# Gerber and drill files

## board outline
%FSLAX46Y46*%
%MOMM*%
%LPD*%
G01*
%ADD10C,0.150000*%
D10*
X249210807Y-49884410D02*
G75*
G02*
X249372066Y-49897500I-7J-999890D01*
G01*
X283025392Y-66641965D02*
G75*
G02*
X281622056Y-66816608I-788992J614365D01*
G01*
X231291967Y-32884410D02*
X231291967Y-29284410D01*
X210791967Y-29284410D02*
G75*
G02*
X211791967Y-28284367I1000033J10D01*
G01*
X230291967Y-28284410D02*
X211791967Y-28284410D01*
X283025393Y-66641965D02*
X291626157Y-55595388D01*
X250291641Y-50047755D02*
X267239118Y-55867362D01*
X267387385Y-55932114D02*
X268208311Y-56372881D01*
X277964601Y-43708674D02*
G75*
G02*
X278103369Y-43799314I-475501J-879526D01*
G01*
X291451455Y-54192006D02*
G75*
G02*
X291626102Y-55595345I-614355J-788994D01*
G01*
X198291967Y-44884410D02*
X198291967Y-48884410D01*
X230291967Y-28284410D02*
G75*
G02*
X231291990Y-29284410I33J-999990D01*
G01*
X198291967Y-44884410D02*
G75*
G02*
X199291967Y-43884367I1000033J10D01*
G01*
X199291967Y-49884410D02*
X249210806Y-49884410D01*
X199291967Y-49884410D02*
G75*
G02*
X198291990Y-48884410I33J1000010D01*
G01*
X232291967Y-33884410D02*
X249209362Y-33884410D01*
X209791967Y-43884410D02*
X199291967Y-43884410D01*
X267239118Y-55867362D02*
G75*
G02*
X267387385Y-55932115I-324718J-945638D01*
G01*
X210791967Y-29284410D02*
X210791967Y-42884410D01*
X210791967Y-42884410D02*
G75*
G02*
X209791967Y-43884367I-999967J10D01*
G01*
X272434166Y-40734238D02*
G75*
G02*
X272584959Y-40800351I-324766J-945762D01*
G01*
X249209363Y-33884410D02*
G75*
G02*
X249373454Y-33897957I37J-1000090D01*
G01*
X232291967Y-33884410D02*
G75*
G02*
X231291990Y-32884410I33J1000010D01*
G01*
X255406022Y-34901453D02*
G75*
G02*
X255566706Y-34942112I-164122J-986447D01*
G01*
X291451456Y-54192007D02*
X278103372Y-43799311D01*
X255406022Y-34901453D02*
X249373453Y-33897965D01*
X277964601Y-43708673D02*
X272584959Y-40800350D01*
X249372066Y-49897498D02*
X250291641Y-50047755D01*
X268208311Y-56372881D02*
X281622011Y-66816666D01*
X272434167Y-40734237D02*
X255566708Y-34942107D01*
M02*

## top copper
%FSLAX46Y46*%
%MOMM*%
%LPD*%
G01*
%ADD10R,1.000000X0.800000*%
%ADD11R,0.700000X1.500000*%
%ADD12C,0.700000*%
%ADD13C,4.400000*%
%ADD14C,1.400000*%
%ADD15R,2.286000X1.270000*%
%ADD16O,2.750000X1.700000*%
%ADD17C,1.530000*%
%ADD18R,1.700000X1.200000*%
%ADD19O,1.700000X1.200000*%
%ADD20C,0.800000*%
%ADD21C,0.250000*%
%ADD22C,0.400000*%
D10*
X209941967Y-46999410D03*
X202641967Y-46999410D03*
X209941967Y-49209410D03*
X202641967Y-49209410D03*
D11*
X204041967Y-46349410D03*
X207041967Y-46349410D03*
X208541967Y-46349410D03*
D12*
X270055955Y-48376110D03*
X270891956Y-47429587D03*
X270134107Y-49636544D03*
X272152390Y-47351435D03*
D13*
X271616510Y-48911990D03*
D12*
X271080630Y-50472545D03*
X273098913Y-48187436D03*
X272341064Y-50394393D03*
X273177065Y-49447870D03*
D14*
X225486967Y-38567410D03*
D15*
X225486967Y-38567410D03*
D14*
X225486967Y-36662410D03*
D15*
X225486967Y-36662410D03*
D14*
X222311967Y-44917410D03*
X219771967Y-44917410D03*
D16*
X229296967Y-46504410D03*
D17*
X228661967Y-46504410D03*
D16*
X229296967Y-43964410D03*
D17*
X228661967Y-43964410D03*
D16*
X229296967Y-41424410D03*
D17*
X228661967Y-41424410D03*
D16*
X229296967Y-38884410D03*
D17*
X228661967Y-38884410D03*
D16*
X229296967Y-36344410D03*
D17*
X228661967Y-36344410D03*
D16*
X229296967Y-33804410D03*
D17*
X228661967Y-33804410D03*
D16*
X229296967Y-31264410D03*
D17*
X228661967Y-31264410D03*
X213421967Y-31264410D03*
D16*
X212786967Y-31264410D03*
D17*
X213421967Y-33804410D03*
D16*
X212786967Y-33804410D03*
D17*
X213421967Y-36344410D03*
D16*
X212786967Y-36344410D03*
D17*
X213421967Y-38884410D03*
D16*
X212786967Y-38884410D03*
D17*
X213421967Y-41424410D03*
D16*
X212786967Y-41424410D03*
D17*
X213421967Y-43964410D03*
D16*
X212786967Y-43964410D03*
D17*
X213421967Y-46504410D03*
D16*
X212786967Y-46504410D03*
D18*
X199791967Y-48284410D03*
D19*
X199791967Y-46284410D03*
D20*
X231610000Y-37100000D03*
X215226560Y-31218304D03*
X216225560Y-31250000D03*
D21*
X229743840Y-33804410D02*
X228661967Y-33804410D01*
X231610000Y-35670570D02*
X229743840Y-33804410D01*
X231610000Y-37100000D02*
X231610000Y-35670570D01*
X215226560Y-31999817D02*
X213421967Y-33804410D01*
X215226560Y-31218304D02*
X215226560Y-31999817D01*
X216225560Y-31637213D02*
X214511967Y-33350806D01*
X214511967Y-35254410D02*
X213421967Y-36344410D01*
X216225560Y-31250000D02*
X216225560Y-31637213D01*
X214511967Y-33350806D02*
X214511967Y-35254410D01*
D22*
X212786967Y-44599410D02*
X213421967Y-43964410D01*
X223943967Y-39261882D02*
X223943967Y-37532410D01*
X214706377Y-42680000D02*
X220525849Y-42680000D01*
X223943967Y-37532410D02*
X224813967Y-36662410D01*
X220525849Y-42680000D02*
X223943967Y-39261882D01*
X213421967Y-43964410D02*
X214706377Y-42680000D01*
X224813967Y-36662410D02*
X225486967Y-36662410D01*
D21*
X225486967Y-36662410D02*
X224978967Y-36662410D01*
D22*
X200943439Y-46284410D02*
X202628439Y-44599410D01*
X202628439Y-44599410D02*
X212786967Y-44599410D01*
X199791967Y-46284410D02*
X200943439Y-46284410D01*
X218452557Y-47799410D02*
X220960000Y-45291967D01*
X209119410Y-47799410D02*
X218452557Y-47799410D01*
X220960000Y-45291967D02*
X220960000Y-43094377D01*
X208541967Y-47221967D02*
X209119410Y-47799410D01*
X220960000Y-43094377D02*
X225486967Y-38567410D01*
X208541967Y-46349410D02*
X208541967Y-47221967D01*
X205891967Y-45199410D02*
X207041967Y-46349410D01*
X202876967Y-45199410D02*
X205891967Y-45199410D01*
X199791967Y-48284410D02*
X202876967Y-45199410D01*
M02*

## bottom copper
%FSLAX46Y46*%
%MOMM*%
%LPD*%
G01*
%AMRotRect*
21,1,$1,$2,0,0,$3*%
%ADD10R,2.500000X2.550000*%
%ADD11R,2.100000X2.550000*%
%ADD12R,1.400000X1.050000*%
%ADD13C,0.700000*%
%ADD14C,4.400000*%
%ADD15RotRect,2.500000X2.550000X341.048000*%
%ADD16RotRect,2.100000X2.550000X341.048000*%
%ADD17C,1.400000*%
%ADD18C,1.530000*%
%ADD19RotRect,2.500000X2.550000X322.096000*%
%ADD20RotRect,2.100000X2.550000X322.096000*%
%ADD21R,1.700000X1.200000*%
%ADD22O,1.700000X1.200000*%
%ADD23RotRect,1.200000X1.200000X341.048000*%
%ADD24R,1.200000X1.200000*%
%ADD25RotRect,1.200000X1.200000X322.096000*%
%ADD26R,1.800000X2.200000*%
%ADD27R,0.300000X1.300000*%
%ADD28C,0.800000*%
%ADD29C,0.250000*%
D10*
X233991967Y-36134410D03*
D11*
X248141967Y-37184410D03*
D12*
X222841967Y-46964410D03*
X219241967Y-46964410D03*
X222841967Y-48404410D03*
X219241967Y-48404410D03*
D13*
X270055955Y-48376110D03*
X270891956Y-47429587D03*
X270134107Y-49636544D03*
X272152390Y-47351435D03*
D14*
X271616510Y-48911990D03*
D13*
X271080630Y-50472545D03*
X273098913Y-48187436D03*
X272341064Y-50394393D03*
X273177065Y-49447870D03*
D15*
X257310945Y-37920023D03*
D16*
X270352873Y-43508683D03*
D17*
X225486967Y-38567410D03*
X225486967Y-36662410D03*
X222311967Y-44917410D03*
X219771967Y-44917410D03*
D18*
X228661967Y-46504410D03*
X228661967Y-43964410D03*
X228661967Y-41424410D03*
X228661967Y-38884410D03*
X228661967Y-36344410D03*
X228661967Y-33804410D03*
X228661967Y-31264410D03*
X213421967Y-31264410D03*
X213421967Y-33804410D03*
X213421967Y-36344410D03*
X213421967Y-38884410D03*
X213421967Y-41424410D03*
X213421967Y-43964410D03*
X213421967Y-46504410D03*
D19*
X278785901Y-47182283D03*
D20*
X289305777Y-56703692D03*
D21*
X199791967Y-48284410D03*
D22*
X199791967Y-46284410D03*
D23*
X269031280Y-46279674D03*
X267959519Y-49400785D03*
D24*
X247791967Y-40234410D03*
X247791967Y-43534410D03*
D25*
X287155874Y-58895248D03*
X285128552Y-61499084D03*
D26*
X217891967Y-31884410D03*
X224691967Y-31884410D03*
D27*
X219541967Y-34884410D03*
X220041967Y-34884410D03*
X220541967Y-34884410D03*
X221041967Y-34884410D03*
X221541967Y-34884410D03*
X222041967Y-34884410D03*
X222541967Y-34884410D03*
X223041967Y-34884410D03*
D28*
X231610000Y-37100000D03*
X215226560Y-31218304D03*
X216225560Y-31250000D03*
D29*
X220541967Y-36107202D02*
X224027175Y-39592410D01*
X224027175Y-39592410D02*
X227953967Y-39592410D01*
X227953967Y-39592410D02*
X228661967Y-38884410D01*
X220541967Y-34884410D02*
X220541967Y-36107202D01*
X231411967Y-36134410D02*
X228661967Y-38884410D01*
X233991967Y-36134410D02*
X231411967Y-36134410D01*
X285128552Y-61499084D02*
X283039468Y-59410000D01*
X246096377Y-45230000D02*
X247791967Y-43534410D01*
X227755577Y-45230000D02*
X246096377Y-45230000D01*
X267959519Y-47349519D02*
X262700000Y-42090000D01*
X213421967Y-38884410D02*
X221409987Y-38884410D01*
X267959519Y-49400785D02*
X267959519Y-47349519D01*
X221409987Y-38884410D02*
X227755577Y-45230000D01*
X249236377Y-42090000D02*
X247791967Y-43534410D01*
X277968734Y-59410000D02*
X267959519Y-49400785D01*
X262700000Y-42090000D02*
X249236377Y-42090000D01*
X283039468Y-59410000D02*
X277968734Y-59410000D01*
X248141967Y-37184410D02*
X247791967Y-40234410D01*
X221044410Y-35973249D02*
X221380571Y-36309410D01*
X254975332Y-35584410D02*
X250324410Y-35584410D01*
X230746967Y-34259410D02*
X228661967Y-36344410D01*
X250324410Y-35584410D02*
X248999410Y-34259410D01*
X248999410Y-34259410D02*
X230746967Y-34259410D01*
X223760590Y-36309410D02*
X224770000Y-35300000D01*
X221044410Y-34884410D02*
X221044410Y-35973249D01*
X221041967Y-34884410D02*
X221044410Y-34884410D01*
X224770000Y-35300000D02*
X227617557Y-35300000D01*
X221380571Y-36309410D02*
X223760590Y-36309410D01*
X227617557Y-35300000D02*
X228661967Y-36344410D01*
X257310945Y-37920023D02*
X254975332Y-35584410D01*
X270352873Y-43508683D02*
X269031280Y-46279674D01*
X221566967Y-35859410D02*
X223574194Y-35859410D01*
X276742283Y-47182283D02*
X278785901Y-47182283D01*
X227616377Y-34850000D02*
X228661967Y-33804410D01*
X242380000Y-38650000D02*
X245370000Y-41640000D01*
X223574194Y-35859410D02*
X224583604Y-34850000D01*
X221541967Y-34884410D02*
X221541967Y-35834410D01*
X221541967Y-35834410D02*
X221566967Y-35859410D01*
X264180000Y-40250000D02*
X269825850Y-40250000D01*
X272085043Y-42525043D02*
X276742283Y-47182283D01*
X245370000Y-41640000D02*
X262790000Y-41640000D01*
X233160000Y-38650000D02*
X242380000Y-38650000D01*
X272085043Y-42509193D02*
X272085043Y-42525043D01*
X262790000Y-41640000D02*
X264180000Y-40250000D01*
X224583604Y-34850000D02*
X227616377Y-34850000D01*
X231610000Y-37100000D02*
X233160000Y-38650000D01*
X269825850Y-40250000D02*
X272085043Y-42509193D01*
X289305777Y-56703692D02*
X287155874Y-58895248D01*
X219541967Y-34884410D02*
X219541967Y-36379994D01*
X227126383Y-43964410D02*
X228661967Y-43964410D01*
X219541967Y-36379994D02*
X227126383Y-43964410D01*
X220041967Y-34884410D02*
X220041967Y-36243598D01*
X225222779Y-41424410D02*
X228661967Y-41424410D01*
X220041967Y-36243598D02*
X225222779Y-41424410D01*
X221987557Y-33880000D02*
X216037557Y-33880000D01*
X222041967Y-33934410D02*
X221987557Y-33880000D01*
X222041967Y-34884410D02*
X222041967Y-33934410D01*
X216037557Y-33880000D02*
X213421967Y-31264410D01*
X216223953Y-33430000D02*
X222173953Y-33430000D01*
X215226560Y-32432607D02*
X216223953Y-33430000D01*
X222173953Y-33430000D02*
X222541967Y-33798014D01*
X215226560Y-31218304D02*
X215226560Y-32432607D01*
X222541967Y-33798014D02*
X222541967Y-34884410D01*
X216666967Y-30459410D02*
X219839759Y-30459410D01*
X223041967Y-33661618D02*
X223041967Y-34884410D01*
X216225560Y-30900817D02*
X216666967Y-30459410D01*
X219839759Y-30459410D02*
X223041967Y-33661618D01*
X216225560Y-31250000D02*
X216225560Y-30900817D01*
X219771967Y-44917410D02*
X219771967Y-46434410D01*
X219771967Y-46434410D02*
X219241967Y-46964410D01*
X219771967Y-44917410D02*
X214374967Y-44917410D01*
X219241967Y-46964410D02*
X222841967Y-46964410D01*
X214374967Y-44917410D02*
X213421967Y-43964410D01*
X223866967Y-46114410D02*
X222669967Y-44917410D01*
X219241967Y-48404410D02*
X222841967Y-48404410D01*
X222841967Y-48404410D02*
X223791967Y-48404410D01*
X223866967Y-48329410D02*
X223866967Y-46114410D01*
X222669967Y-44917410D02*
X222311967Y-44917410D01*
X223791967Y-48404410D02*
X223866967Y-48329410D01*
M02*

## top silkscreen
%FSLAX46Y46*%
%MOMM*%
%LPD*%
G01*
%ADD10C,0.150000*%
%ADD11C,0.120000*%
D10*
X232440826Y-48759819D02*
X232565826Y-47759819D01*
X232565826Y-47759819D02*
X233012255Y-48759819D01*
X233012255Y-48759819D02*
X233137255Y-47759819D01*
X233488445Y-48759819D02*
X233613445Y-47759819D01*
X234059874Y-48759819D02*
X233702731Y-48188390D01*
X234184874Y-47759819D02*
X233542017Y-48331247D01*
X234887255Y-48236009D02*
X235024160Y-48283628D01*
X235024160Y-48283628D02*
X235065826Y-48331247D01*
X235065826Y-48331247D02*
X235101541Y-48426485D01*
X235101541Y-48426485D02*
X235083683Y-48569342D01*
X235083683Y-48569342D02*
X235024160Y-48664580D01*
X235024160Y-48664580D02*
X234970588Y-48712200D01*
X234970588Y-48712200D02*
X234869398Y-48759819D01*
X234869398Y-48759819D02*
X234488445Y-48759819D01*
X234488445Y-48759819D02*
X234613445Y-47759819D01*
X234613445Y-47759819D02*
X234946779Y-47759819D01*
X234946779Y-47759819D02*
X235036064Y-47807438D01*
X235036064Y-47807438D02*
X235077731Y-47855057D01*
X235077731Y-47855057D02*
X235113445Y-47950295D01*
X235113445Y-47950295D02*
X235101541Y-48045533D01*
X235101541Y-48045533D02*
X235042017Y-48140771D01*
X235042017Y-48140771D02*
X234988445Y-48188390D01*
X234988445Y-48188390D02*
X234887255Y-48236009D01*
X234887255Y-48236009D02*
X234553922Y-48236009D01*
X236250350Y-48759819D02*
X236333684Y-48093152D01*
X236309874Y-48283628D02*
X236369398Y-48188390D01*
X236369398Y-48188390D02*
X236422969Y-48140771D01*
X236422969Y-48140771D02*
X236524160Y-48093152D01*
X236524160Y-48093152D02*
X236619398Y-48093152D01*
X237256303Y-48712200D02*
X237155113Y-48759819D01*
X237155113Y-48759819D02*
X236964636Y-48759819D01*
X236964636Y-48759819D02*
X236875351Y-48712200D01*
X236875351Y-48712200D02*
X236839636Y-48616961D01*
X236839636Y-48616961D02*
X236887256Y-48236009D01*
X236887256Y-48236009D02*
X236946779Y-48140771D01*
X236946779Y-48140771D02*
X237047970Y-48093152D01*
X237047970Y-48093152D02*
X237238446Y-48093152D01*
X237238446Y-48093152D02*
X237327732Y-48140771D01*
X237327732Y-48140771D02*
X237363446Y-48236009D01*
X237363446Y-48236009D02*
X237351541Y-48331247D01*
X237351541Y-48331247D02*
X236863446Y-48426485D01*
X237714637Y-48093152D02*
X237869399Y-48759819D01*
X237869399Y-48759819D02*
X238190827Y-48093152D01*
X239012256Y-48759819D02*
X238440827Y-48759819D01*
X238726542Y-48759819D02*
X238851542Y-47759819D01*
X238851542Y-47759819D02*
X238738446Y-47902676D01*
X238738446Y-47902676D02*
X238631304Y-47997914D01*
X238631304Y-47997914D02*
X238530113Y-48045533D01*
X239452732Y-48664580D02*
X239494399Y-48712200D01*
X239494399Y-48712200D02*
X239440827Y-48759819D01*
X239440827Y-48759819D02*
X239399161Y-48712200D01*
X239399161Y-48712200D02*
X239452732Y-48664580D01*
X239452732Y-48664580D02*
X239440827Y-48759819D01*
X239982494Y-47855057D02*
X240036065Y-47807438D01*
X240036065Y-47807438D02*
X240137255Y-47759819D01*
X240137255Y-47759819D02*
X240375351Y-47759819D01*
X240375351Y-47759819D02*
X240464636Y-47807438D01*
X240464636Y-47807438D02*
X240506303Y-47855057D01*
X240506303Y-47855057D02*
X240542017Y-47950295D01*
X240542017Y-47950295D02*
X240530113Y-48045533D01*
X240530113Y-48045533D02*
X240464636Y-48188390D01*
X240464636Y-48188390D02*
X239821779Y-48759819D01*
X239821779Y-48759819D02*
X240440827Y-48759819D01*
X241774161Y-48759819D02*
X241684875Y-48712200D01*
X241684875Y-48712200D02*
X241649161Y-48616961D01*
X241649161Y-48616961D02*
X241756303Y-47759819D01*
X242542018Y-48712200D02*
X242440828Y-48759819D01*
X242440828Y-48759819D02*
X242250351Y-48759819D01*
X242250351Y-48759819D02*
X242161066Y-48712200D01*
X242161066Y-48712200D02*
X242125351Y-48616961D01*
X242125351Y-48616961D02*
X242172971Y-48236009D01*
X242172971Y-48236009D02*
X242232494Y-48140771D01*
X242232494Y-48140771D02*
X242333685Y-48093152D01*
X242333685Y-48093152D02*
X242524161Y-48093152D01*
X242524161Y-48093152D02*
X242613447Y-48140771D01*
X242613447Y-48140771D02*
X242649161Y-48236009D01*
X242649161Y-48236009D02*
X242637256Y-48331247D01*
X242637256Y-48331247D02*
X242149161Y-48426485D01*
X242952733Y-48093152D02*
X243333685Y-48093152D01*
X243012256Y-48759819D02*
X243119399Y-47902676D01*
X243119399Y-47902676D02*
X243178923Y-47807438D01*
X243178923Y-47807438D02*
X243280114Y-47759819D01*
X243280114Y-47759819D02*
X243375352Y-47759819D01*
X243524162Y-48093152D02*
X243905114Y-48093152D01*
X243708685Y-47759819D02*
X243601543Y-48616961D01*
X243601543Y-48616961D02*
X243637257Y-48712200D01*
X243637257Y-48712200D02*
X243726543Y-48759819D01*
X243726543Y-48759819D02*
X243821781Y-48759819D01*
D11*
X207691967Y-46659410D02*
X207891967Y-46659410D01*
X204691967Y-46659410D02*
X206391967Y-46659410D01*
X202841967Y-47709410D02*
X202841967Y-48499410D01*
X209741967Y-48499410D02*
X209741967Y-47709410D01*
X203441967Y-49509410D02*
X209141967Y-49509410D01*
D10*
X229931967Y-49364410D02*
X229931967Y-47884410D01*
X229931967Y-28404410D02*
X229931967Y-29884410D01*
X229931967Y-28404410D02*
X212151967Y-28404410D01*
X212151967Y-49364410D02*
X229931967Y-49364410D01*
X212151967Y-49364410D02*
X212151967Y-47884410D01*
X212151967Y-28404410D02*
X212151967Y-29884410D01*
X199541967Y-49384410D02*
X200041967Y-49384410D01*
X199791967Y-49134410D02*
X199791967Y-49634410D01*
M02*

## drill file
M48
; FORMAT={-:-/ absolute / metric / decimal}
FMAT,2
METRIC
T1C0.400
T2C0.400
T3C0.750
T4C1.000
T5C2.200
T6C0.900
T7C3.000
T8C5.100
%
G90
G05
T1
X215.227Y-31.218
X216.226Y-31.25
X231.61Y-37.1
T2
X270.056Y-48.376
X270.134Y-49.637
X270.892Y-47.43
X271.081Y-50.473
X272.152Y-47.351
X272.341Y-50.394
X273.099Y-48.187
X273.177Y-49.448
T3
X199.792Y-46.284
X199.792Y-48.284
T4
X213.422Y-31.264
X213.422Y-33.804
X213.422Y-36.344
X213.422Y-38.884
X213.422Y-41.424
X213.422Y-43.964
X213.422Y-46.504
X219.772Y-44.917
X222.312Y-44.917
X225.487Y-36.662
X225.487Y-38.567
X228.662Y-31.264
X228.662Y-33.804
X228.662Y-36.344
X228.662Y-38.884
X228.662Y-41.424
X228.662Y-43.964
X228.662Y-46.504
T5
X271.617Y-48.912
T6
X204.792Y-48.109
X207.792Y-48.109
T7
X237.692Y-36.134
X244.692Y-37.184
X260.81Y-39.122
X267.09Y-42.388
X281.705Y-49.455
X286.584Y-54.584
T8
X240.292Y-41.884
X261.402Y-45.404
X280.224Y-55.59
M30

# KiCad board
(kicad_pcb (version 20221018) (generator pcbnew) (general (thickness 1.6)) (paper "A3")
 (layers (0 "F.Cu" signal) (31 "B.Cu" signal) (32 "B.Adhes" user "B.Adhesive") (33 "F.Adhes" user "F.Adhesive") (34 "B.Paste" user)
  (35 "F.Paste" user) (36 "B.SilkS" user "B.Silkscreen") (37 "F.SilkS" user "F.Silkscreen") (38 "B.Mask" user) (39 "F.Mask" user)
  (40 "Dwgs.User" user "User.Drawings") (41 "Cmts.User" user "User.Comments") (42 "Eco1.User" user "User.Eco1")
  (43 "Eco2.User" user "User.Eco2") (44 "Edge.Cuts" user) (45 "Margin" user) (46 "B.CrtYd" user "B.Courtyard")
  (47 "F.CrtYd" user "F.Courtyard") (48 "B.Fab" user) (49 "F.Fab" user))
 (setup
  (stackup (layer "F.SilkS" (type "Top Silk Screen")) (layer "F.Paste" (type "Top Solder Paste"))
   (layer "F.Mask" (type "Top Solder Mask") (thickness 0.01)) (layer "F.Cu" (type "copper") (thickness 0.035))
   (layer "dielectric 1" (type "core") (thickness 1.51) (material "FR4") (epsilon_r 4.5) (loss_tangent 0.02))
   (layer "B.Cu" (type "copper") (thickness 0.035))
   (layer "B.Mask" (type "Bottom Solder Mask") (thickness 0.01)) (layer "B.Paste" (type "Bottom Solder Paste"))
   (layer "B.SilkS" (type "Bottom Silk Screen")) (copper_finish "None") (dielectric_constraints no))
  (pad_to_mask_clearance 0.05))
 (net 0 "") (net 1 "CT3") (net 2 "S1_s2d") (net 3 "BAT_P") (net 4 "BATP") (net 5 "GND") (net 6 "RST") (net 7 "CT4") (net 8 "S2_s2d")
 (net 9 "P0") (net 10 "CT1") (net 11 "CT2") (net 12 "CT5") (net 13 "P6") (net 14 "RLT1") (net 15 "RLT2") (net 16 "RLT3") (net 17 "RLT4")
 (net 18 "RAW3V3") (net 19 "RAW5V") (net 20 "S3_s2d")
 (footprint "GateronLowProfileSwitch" (layer "F.Cu") (at 240.291967 41.88441)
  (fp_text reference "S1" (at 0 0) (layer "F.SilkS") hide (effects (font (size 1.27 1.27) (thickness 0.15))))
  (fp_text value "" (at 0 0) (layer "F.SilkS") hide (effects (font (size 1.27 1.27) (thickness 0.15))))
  (pad "" np_thru_hole circle (at -2.6 -5.75) (size 3 3) (drill 3) (layers "*.Cu" "*.Mask"))
  (pad "" np_thru_hole circle (at 0 0) (size 5.1 5.1) (drill 5.1) (layers "*.Cu" "*.Mask"))
  (pad "" np_thru_hole circle (at 4.4 -4.7) (size 3 3) (drill 3) (layers "*.Cu" "*.Mask"))
  (pad "1" smd rect (at -6.3 -5.75) (size 2.5 2.55) (layers "B.Cu" "B.Paste" "B.Mask") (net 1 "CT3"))
  (pad "2" smd rect (at 7.85 -4.7) (size 2.1 2.55) (layers "B.Cu" "B.Paste" "B.Mask") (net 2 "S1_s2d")))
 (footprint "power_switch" (layer "F.Cu") (at 206.291967 48.08441 -90)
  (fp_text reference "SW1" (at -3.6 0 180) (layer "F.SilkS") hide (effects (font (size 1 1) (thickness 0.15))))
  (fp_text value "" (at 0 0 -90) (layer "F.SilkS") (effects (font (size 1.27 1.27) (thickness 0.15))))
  (fp_line (start -1.425 -1.4) (end -1.425 -1.6) (stroke (width 0.12) (type solid)) (layer "F.SilkS"))
  (fp_line (start -1.425 1.6) (end -1.425 -0.1) (stroke (width 0.12) (type solid)) (layer "F.SilkS"))
  (fp_line (start -0.375 3.45) (end 0.415 3.45) (stroke (width 0.12) (type solid)) (layer "F.SilkS"))
  (fp_line (start 0.415 -3.45) (end -0.375 -3.45) (stroke (width 0.12) (type solid)) (layer "F.SilkS"))
  (fp_line (start 1.425 2.85) (end 1.425 -2.85) (stroke (width 0.12) (type solid)) (layer "F.SilkS"))
  (pad "" smd rect (at -1.085 -3.65) (size 1 0.8) (layers "F.Cu" "F.Paste" "F.Mask"))
  (pad "" smd rect (at -1.085 3.65) (size 1 0.8) (layers "F.Cu" "F.Paste" "F.Mask"))
  (pad "" np_thru_hole circle (at 0.025 -1.5) (size 0.9 0.9) (drill 0.9) (layers "*.Cu" "*.Mask"))
  (pad "" np_thru_hole circle (at 0.025 1.5) (size 0.9 0.9) (drill 0.9) (layers "*.Cu" "*.Mask"))
  (pad "" smd rect (at 1.125 -3.65) (size 1 0.8) (layers "F.Cu" "F.Paste" "F.Mask"))
  (pad "" smd rect (at 1.125 3.65) (size 1 0.8) (layers "F.Cu" "F.Paste" "F.Mask"))
  (pad "1" smd rect (at -1.735 2.25) (size 0.7 1.5) (layers "F.Cu" "F.Paste" "F.Mask"))
  (pad "2" smd rect (at -1.735 -0.75) (size 0.7 1.5) (layers "F.Cu" "F.Paste" "F.Mask") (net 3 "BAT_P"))
  (pad "3" smd rect (at -1.735 -2.25) (size 0.7 1.5) (layers "F.Cu" "F.Paste" "F.Mask") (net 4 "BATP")))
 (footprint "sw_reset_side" (layer "F.Cu") (at 221.041967 47.68441 -90)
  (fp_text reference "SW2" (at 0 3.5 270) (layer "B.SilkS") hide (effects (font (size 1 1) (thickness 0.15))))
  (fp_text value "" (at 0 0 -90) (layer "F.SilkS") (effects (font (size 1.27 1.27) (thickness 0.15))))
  (pad "1" smd rect (at -0.72 -1.8 180) (size 1.4 1.05) (layers "B.Cu" "B.Paste" "B.Mask") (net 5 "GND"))
  (pad "1" smd rect (at -0.72 1.8 180) (size 1.4 1.05) (layers "B.Cu" "B.Paste" "B.Mask") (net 5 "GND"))
  (pad "2" smd rect (at 0.72 -1.8 180) (size 1.4 1.05) (layers "B.Cu" "B.Paste" "B.Mask") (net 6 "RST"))
  (pad "2" smd rect (at 0.72 1.8 180) (size 1.4 1.05) (layers "B.Cu" "B.Paste" "B.Mask") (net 6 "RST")))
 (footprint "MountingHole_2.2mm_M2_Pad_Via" (layer "F.Cu") (at 271.61651 48.91199 -18.952)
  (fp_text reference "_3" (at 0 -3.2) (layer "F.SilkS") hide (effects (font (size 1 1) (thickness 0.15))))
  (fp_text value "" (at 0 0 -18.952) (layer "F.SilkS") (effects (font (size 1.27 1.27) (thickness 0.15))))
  (pad "1" thru_hole circle (at -1.65 0) (size 0.7 0.7) (drill 0.4) (layers "*.Cu" "*.Mask"))
  (pad "1" thru_hole circle (at -1.166726 -1.166726) (size 0.7 0.7) (drill 0.4) (layers "*.Cu" "*.Mask"))
  (pad "1" thru_hole circle (at -1.166726 1.166726) (size 0.7 0.7) (drill 0.4) (layers "*.Cu" "*.Mask"))
  (pad "1" thru_hole circle (at 0 -1.65) (size 0.7 0.7) (drill 0.4) (layers "*.Cu" "*.Mask"))
  (pad "1" thru_hole circle (at 0 0) (size 4.4 4.4) (drill 2.2) (layers "*.Cu" "*.Mask"))
  (pad "1" thru_hole circle (at 0 1.65) (size 0.7 0.7) (drill 0.4) (layers "*.Cu" "*.Mask"))
  (pad "1" thru_hole circle (at 1.166726 -1.166726) (size 0.7 0.7) (drill 0.4) (layers "*.Cu" "*.Mask"))
  (pad "1" thru_hole circle (at 1.166726 1.166726) (size 0.7 0.7) (drill 0.4) (layers "*.Cu" "*.Mask"))
  (pad "1" thru_hole circle (at 1.65 0) (size 0.7 0.7) (drill 0.4) (layers "*.Cu" "*.Mask")))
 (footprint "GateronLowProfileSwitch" (layer "F.Cu") (at 261.401967 45.40441 -18.952)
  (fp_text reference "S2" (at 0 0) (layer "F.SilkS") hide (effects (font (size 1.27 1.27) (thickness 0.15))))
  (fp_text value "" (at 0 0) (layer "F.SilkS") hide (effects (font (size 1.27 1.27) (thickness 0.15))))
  (pad "" np_thru_hole circle (at -2.6 -5.75) (size 3 3) (drill 3) (layers "*.Cu" "*.Mask"))
  (pad "" np_thru_hole circle (at 0 0) (size 5.1 5.1) (drill 5.1) (layers "*.Cu" "*.Mask"))
  (pad "" np_thru_hole circle (at 4.4 -4.7) (size 3 3) (drill 3) (layers "*.Cu" "*.Mask"))
  (pad "1" smd rect (at -6.3 -5.75 341.048) (size 2.5 2.55) (layers "B.Cu" "B.Paste" "B.Mask") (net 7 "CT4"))
  (pad "2" smd rect (at 7.85 -4.7 341.048) (size 2.1 2.55) (layers "B.Cu" "B.Paste" "B.Mask") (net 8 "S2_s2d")))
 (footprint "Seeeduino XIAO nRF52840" (layer "F.Cu") (at 221.041967 38.88441 180)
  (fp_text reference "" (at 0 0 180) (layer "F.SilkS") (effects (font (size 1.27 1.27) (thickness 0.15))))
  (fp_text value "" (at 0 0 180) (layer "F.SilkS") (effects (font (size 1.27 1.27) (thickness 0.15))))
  (fp_line (start -8.89 -10.48) (end -8.89 -9) (stroke (width 0.15) (type solid)) (layer "F.SilkS"))
  (fp_line (start -8.89 10.48) (end -8.89 9) (stroke (width 0.15) (type solid)) (layer "F.SilkS"))
  (fp_line (start -8.89 10.48) (end 8.89 10.48) (stroke (width 0.15) (type solid)) (layer "F.SilkS"))
  (fp_line (start 8.89 -10.48) (end -8.89 -10.48) (stroke (width 0.15) (type solid)) (layer "F.SilkS"))
  (fp_line (start 8.89 -10.48) (end 8.89 -9) (stroke (width 0.15) (type solid)) (layer "F.SilkS"))
  (fp_line (start 8.89 10.48) (end 8.89 9) (stroke (width 0.15) (type solid)) (layer "F.SilkS"))
  (pad "" thru_hole circle (at -4.445 0.317) (size 1.4 1.4) (drill 1) (layers "*.Cu" "*.Mask") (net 4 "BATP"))
  (pad "" smd rect (at -4.445 0.317 180) (size 2.286 1.27) (layers "F.Cu" "F.Paste" "F.Mask") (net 4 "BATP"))
  (pad "" thru_hole circle (at -4.445 2.222) (size 1.4 1.4) (drill 1) (layers "*.Cu" "*.Mask") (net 5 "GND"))
  (pad "" smd rect (at -4.445 2.222 180) (size 2.286 1.27) (layers "F.Cu" "F.Paste" "F.Mask") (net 5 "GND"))
  (pad "" thru_hole circle (at -1.27 -6.033) (size 1.4 1.4) (drill 1) (layers "*.Cu" "*.Mask") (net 6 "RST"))
  (pad "" thru_hole circle (at 1.27 -6.033) (size 1.4 1.4) (drill 1) (layers "*.Cu" "*.Mask") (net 5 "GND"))
  (pad "1" smd oval (at -8.255 -7.62 180) (size 2.75 1.7) (layers "F.Cu" "F.Paste" "F.Mask") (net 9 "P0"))
  (pad "1" thru_hole circle (at -7.62 -7.62) (size 1.53 1.53) (drill 1) (layers "*.Cu" "*.Mask") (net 9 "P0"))
  (pad "2" smd oval (at -8.255 -5.08 180) (size 2.75 1.7) (layers "F.Cu" "F.Paste" "F.Mask") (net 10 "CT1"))
  (pad "2" thru_hole circle (at -7.62 -5.08) (size 1.53 1.53) (drill 1) (layers "*.Cu" "*.Mask") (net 10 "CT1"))
  (pad "3" smd oval (at -8.255 -2.54 180) (size 2.75 1.7) (layers "F.Cu" "F.Paste" "F.Mask") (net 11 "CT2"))
  (pad "3" thru_hole circle (at -7.62 -2.54) (size 1.53 1.53) (drill 1) (layers "*.Cu" "*.Mask") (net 11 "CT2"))
  (pad "4" smd oval (at -8.255 0 180) (size 2.75 1.7) (layers "F.Cu" "F.Paste" "F.Mask") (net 1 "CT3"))
  (pad "4" thru_hole circle (at -7.62 0) (size 1.53 1.53) (drill 1) (layers "*.Cu" "*.Mask") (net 1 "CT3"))
  (pad "5" smd oval (at -8.255 2.54 180) (size 2.75 1.7) (layers "F.Cu" "F.Paste" "F.Mask") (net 7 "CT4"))
  (pad "5" thru_hole circle (at -7.62 2.54) (size 1.53 1.53) (drill 1) (layers "*.Cu" "*.Mask") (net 7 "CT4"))
  (pad "6" smd oval (at -8.255 5.08 180) (size 2.75 1.7) (layers "F.Cu" "F.Paste" "F.Mask") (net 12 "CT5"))
  (pad "6" thru_hole circle (at -7.62 5.08) (size 1.53 1.53) (drill 1) (layers "*.Cu" "*.Mask") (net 12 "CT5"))
  (pad "7" smd oval (at -8.255 7.62 180) (size 2.75 1.7) (layers "F.Cu" "F.Paste" "F.Mask") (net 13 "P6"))
  (pad "7" thru_hole circle (at -7.62 7.62) (size 1.53 1.53) (drill 1) (layers "*.Cu" "*.Mask") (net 13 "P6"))
  (pad "8" thru_hole circle (at 7.62 7.62) (size 1.53 1.53) (drill 1) (layers "*.Cu" "*.Mask") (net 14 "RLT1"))
  (pad "8" smd oval (at 8.255 7.62 180) (size 2.75 1.7) (layers "F.Cu" "F.Paste" "F.Mask") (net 14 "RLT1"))
  (pad "9" thru_hole circle (at 7.62 5.08) (size 1.53 1.53) (drill 1) (layers "*.Cu" "*.Mask") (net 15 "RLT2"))
  (pad "9" smd oval (at 8.255 5.08 180) (size 2.75 1.7) (layers "F.Cu" "F.Paste" "F.Mask") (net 15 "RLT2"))
  (pad "10" thru_hole circle (at 7.62 2.54) (size 1.53 1.53) (drill 1) (layers "*.Cu" "*.Mask") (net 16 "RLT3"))
  (pad "10" smd oval (at 8.255 2.54 180) (size 2.75 1.7) (layers "F.Cu" "F.Paste" "F.Mask") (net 16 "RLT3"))
  (pad "11" thru_hole circle (at 7.62 0) (size 1.53 1.53) (drill 1) (layers "*.Cu" "*.Mask") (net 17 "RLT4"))
  (pad "11" smd oval (at 8.255 0 180) (size 2.75 1.7) (layers "F.Cu" "F.Paste" "F.Mask") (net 17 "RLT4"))
  (pad "12" thru_hole circle (at 7.62 -2.54) (size 1.53 1.53) (drill 1) (layers "*.Cu" "*.Mask") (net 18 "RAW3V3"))
  (pad "12" smd oval (at 8.255 -2.54 180) (size 2.75 1.7) (layers "F.Cu" "F.Paste" "F.Mask") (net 18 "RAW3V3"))
  (pad "13" thru_hole circle (at 7.62 -5.08) (size 1.53 1.53) (drill 1) (layers "*.Cu" "*.Mask") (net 5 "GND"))
  (pad "13" smd oval (at 8.255 -5.08 180) (size 2.75 1.7) (layers "F.Cu" "F.Paste" "F.Mask") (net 5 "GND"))
  (pad "14" thru_hole circle (at 7.62 -7.62) (size 1.53 1.53) (drill 1) (layers "*.Cu" "*.Mask") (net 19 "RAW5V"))
  (pad "14" smd oval (at 8.255 -7.62 180) (size 2.75 1.7) (layers "F.Cu" "F.Paste" "F.Mask") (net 19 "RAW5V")))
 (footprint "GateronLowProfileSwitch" (layer "F.Cu") (at 280.224404 55.589614 -37.904)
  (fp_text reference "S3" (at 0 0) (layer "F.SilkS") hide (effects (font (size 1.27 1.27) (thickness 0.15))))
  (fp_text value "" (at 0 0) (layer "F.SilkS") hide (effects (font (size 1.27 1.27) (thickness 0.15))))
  (pad "" np_thru_hole circle (at -2.6 -5.75) (size 3 3) (drill 3) (layers "*.Cu" "*.Mask"))
  (pad "" np_thru_hole circle (at 0 0) (size 5.1 5.1) (drill 5.1) (layers "*.Cu" "*.Mask"))
  (pad "" np_thru_hole circle (at 4.4 -4.7) (size 3 3) (drill 3) (layers "*.Cu" "*.Mask"))
  (pad "1" smd rect (at -6.3 -5.75 322.096) (size 2.5 2.55) (layers "B.Cu" "B.Paste" "B.Mask") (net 12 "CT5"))
  (pad "2" smd rect (at 7.85 -4.7 322.096) (size 2.1 2.55) (layers "B.Cu" "B.Paste" "B.Mask") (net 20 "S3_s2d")))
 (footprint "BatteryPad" (layer "F.Cu") (at 199.791967 47.28441 90)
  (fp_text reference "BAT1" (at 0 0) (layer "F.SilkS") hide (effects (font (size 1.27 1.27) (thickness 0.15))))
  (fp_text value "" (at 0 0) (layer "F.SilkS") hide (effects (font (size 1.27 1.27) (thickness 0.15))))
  (fp_line (start -2.1 -0.25) (end -2.1 0.25) (stroke (width 0.15) (type solid)) (layer "F.SilkS"))
  (fp_line (start -1.85 0) (end -2.35 0) (stroke (width 0.15) (type solid)) (layer "F.SilkS"))
  (pad "1" thru_hole rect (at -1 0 90) (size 1.2 1.7) (drill 0.75) (layers "*.Cu" "*.Mask") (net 3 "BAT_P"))
  (pad "2" thru_hole oval (at 1 0 90) (size 1.2 1.7) (drill 0.75) (layers "*.Cu" "*.Mask") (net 5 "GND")))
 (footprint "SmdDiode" (layer "B.Cu") (at 261.401967 45.40441 -18.952)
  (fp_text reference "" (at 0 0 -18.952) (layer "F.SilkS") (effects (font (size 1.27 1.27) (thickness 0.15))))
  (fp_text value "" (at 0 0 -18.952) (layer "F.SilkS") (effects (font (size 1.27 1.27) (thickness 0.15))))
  (pad "1" smd rect (at 7.5 -1.65 341.048) (size 1.2 1.2) (layers "B.Cu" "B.Paste" "B.Mask") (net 8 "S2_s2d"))
  (pad "2" smd rect (at 7.5 1.65 341.048) (size 1.2 1.2) (layers "B.Cu" "B.Paste" "B.Mask") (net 17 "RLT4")))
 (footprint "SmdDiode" (layer "B.Cu") (at 240.291967 41.88441)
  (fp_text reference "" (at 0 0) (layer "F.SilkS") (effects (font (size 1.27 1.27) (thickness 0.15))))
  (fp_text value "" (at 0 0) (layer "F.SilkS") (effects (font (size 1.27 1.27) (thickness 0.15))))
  (pad "1" smd rect (at 7.5 -1.65) (size 1.2 1.2) (layers "B.Cu" "B.Paste" "B.Mask") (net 2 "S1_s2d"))
  (pad "2" smd rect (at 7.5 1.65) (size 1.2 1.2) (layers "B.Cu" "B.Paste" "B.Mask") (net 17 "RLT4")))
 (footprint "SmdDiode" (layer "B.Cu") (at 280.224404 55.589614 -37.904)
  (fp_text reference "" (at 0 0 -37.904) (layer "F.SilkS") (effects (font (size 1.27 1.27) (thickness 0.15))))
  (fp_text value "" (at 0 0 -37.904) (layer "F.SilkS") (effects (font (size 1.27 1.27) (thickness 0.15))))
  (pad "1" smd rect (at 7.5 -1.65 322.096) (size 1.2 1.2) (layers "B.Cu" "B.Paste" "B.Mask") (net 20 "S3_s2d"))
  (pad "2" smd rect (at 7.5 1.65 322.096) (size 1.2 1.2) (layers "B.Cu" "B.Paste" "B.Mask") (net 17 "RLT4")))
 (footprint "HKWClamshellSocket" (layer "B.Cu") (at 221.291967 31.88441)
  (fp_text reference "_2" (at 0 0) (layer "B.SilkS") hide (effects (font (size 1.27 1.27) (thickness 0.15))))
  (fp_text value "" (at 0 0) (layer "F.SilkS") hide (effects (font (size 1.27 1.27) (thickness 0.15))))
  (pad "" smd rect (at -3.4 0) (size 1.8 2.2) (layers "B.Cu" "B.Paste" "B.Mask"))
  (pad "" smd rect (at 3.4 0) (size 1.8 2.2) (layers "B.Cu" "B.Paste" "B.Mask"))
  (pad "1" smd rect (at -1.75 3) (size 0.3 1.3) (layers "B.Cu" "B.Paste" "B.Mask") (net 10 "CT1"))
  (pad "2" smd rect (at -1.25 3) (size 0.3 1.3) (layers "B.Cu" "B.Paste" "B.Mask") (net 11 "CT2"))
  (pad "3" smd rect (at -0.75 3) (size 0.3 1.3) (layers "B.Cu" "B.Paste" "B.Mask") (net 1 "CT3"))
  (pad "4" smd rect (at -0.25 3) (size 0.3 1.3) (layers "B.Cu" "B.Paste" "B.Mask") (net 7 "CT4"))
  (pad "5" smd rect (at 0.25 3) (size 0.3 1.3) (layers "B.Cu" "B.Paste" "B.Mask") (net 12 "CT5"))
  (pad "6" smd rect (at 0.75 3) (size 0.3 1.3) (layers "B.Cu" "B.Paste" "B.Mask") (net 14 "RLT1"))
  (pad "7" smd rect (at 1.25 3) (size 0.3 1.3) (layers "B.Cu" "B.Paste" "B.Mask") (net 15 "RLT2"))
  (pad "8" smd rect (at 1.75 3) (size 0.3 1.3) (layers "B.Cu" "B.Paste" "B.Mask") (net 16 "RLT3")))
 (gr_arc (start 249.210807 49.88441) (mid 249.291702 49.887687) (end 249.372066 49.897498) (stroke (width 0.15) (type solid))
  (layer "Edge.Cuts"))
 (gr_arc (start 283.025392 66.641965) (mid 282.359883 67.019965) (end 281.622011 66.816666) (stroke (width 0.15) (type solid))
  (layer "Edge.Cuts"))
 (gr_line (start 231.291967 32.88441) (end 231.291967 29.28441) (stroke (width 0.15) (type solid)) (layer "Edge.Cuts"))
 (gr_arc (start 210.791967 29.28441) (mid 211.08486 28.577303) (end 211.791967 28.28441) (stroke (width 0.15) (type solid))
  (layer "Edge.Cuts"))
 (gr_line (start 230.291967 28.28441) (end 211.791967 28.28441) (stroke (width 0.15) (type solid)) (layer "Edge.Cuts"))
 (gr_line (start 283.025393 66.641965) (end 291.626157 55.595388) (stroke (width 0.15) (type solid)) (layer "Edge.Cuts"))
 (gr_line (start 250.291641 50.047755) (end 267.239118 55.867362) (stroke (width 0.15) (type solid)) (layer "Edge.Cuts"))
 (gr_line (start 267.387385 55.932114) (end 268.208311 56.372881) (stroke (width 0.15) (type solid)) (layer "Edge.Cuts"))
 (gr_arc (start 277.964601 43.708674) (mid 278.035868 43.751112) (end 278.103372 43.799311) (stroke (width 0.15) (type solid))
  (layer "Edge.Cuts"))
 (gr_arc (start 291.451455 54.192006) (mid 291.829456 54.857515) (end 291.626157 55.595388) (stroke (width 0.15) (type solid))
  (layer "Edge.Cuts"))
 (gr_line (start 198.291967 44.88441) (end 198.291967 48.88441) (stroke (width 0.15) (type solid)) (layer "Edge.Cuts"))
 (gr_arc (start 230.291967 28.28441) (mid 230.999074 28.577303) (end 231.291967 29.28441) (stroke (width 0.15) (type solid))
  (layer "Edge.Cuts"))
 (gr_arc (start 198.291967 44.88441) (mid 198.58486 44.177303) (end 199.291967 43.88441) (stroke (width 0.15) (type solid))
  (layer "Edge.Cuts"))
 (gr_line (start 199.291967 49.88441) (end 249.210806 49.88441) (stroke (width 0.15) (type solid)) (layer "Edge.Cuts"))
 (gr_arc (start 199.291967 49.88441) (mid 198.58486 49.591517) (end 198.291967 48.88441) (stroke (width 0.15) (type solid))
  (layer "Edge.Cuts"))
 (gr_line (start 232.291967 33.88441) (end 249.209362 33.88441) (stroke (width 0.15) (type solid)) (layer "Edge.Cuts"))
 (gr_line (start 209.791967 43.88441) (end 199.291967 43.88441) (stroke (width 0.15) (type solid)) (layer "Edge.Cuts"))
 (gr_arc (start 267.239118 55.867362) (mid 267.314563 55.896734) (end 267.387385 55.932114) (stroke (width 0.15) (type solid))
  (layer "Edge.Cuts"))
 (gr_line (start 210.791967 29.28441) (end 210.791967 42.88441) (stroke (width 0.15) (type solid)) (layer "Edge.Cuts"))
 (gr_arc (start 210.791967 42.88441) (mid 210.499074 43.591517) (end 209.791967 43.88441) (stroke (width 0.15) (type solid))
  (layer "Edge.Cuts"))
 (gr_arc (start 272.434166 40.734238) (mid 272.510925 40.764185) (end 272.584959 40.80035) (stroke (width 0.15) (type solid))
  (layer "Edge.Cuts"))
 (gr_arc (start 249.209363 33.88441) (mid 249.291687 33.887805) (end 249.373453 33.897965) (stroke (width 0.15) (type solid))
  (layer "Edge.Cuts"))
 (gr_arc (start 232.291967 33.88441) (mid 231.58486 33.591517) (end 231.291967 32.88441) (stroke (width 0.15) (type solid))
  (layer "Edge.Cuts"))
 (gr_arc (start 255.406022 34.901453) (mid 255.487209 34.918445) (end 255.566708 34.942107) (stroke (width 0.15) (type solid))
  (layer "Edge.Cuts"))
 (gr_line (start 291.451456 54.192007) (end 278.103372 43.799311) (stroke (width 0.15) (type solid)) (layer "Edge.Cuts"))
 (gr_line (start 255.406022 34.901453) (end 249.373453 33.897965) (stroke (width 0.15) (type solid)) (layer "Edge.Cuts"))
 (gr_line (start 277.964601 43.708673) (end 272.584959 40.80035) (stroke (width 0.15) (type solid)) (layer "Edge.Cuts"))
 (gr_line (start 249.372066 49.897498) (end 250.291641 50.047755) (stroke (width 0.15) (type solid)) (layer "Edge.Cuts"))
 (gr_line (start 268.208311 56.372881) (end 281.622011 66.816666) (stroke (width 0.15) (type solid)) (layer "Edge.Cuts"))
 (gr_line (start 272.434167 40.734237) (end 255.566708 34.942107) (stroke (width 0.15) (type solid)) (layer "Edge.Cuts"))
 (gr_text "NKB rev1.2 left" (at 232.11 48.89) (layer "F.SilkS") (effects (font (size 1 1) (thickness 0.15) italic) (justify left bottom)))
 (segment (start 220.541967 36.107202) (end 224.027175 39.59241) (width 0.25) (layer "B.Cu") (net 1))
 (segment (start 224.027175 39.59241) (end 227.953967 39.59241) (width 0.25) (layer "B.Cu") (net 1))
 (segment (start 227.953967 39.59241) (end 228.661967 38.88441) (width 0.25) (layer "B.Cu") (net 1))
 (segment (start 220.541967 34.88441) (end 220.541967 36.107202) (width 0.25) (layer "B.Cu") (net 1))
 (segment (start 231.411967 36.13441) (end 228.661967 38.88441) (width 0.25) (layer "B.Cu") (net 1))
 (segment (start 233.991967 36.13441) (end 231.411967 36.13441) (width 0.25) (layer "B.Cu") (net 1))
 (segment (start 285.128552 61.499084) (end 283.039468 59.41) (width 0.25) (layer "B.Cu") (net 17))
 (segment (start 246.096377 45.23) (end 247.791967 43.53441) (width 0.25) (layer "B.Cu") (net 17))
 (segment (start 227.755577 45.23) (end 246.096377 45.23) (width 0.25) (layer "B.Cu") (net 17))
 (segment (start 267.959519 47.349519) (end 262.7 42.09) (width 0.25) (layer "B.Cu") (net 17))
 (segment (start 213.421967 38.88441) (end 221.409987 38.88441) (width 0.25) (layer "B.Cu") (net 17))
 (segment (start 267.959519 49.400785) (end 267.959519 47.349519) (width 0.25) (layer "B.Cu") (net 17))
 (segment (start 221.409987 38.88441) (end 227.755577 45.23) (width 0.25) (layer "B.Cu") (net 17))
 (segment (start 249.236377 42.09) (end 247.791967 43.53441) (width 0.25) (layer "B.Cu") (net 17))
 (segment (start 277.968734 59.41) (end 267.959519 49.400785) (width 0.25) (layer "B.Cu") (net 17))
 (segment (start 262.7 42.09) (end 249.236377 42.09) (width 0.25) (layer "B.Cu") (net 17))
 (segment (start 283.039468 59.41) (end 277.968734 59.41) (width 0.25) (layer "B.Cu") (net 17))
 (segment (start 248.141967 37.18441) (end 247.791967 40.23441) (width 0.25) (layer "B.Cu") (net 2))
 (segment (start 221.04441 35.973249) (end 221.380571 36.30941) (width 0.25) (layer "B.Cu") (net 7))
 (segment (start 254.975332 35.58441) (end 250.32441 35.58441) (width 0.25) (layer "B.Cu") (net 7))
 (segment (start 230.746967 34.25941) (end 228.661967 36.34441) (width 0.25) (layer "B.Cu") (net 7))
 (segment (start 250.32441 35.58441) (end 248.99941 34.25941) (width 0.25) (layer "B.Cu") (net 7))
 (segment (start 248.99941 34.25941) (end 230.746967 34.25941) (width 0.25) (layer "B.Cu") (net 7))
 (segment (start 223.76059 36.30941) (end 224.77 35.3) (width 0.25) (layer "B.Cu") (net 7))
 (segment (start 221.04441 34.88441) (end 221.04441 35.973249) (width 0.25) (layer "B.Cu") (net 7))
 (segment (start 221.041967 34.88441) (end 221.04441 34.88441) (width 0.25) (layer "B.Cu") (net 7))
 (segment (start 224.77 35.3) (end 227.617557 35.3) (width 0.25) (layer "B.Cu") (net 7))
 (segment (start 221.380571 36.30941) (end 223.76059 36.30941) (width 0.25) (layer "B.Cu") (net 7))
 (segment (start 227.617557 35.3) (end 228.661967 36.34441) (width 0.25) (layer "B.Cu") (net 7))
 (segment (start 257.310945 37.920023) (end 254.975332 35.58441) (width 0.25) (layer "B.Cu") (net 7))
 (segment (start 270.352873 43.508683) (end 269.03128 46.279674) (width 0.25) (layer "B.Cu") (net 8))
 (segment (start 229.74384 33.80441) (end 228.661967 33.80441) (width 0.25) (layer "F.Cu") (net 12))
 (segment (start 231.61 35.67057) (end 229.74384 33.80441) (width 0.25) (layer "F.Cu") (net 12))
 (segment (start 231.61 37.1) (end 231.61 35.67057) (width 0.25) (layer "F.Cu") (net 12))
 (via (at 231.61 37.1) (size 0.8) (drill 0.4) (layers "F.Cu" "B.Cu") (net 12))
 (segment (start 221.566967 35.85941) (end 223.574194 35.85941) (width 0.25) (layer "B.Cu") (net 12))
 (segment (start 276.742283 47.182283) (end 278.785901 47.182283) (width 0.25) (layer "B.Cu") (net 12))
 (segment (start 227.616377 34.85) (end 228.661967 33.80441) (width 0.25) (layer "B.Cu") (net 12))
 (segment (start 242.38 38.65) (end 245.37 41.64) (width 0.25) (layer "B.Cu") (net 12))
 (segment (start 223.574194 35.85941) (end 224.583604 34.85) (width 0.25) (layer "B.Cu") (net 12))
 (segment (start 221.541967 34.88441) (end 221.541967 35.83441) (width 0.25) (layer "B.Cu") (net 12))
 (segment (start 221.541967 35.83441) (end 221.566967 35.85941) (width 0.25) (layer "B.Cu") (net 12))
 (segment (start 264.18 40.25) (end 269.82585 40.25) (width 0.25) (layer "B.Cu") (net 12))
 (segment (start 272.085043 42.525043) (end 276.742283 47.182283) (width 0.25) (layer "B.Cu") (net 12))
 (segment (start 245.37 41.64) (end 262.79 41.64) (width 0.25) (layer "B.Cu") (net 12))
 (segment (start 233.16 38.65) (end 242.38 38.65) (width 0.25) (layer "B.Cu") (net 12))
 (segment (start 272.085043 42.509193) (end 272.085043 42.525043) (width 0.25) (layer "B.Cu") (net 12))
 (segment (start 262.79 41.64) (end 264.18 40.25) (width 0.25) (layer "B.Cu") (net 12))
 (segment (start 224.583604 34.85) (end 227.616377 34.85) (width 0.25) (layer "B.Cu") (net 12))
 (segment (start 231.61 37.1) (end 233.16 38.65) (width 0.25) (layer "B.Cu") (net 12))
 (segment (start 269.82585 40.25) (end 272.085043 42.509193) (width 0.25) (layer "B.Cu") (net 12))
 (segment (start 289.305777 56.703692) (end 287.155874 58.895248) (width 0.25) (layer "B.Cu") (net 20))
 (segment (start 219.541967 34.88441) (end 219.541967 36.379994) (width 0.25) (layer "B.Cu") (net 10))
 (segment (start 227.126383 43.96441) (end 228.661967 43.96441) (width 0.25) (layer "B.Cu") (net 10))
 (segment (start 219.541967 36.379994) (end 227.126383 43.96441) (width 0.25) (layer "B.Cu") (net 10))
 (segment (start 220.041967 34.88441) (end 220.041967 36.243598) (width 0.25) (layer "B.Cu") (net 11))
 (segment (start 225.222779 41.42441) (end 228.661967 41.42441) (width 0.25) (layer "B.Cu") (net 11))
 (segment (start 220.041967 36.243598) (end 225.222779 41.42441) (width 0.25) (layer "B.Cu") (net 11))
 (segment (start 221.987557 33.88) (end 216.037557 33.88) (width 0.25) (layer "B.Cu") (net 14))
 (segment (start 222.041967 33.93441) (end 221.987557 33.88) (width 0.25) (layer "B.Cu") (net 14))
 (segment (start 222.041967 34.88441) (end 222.041967 33.93441) (width 0.25) (layer "B.Cu") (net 14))
 (segment (start 216.037557 33.88) (end 213.421967 31.26441) (width 0.25) (layer "B.Cu") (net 14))
 (segment (start 215.22656 31.999817) (end 213.421967 33.80441) (width 0.25) (layer "F.Cu") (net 15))
 (segment (start 215.22656 31.218304) (end 215.22656 31.999817) (width 0.25) (layer "F.Cu") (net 15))
 (via (at 215.22656 31.218304) (size 0.8) (drill 0.4) (layers "F.Cu" "B.Cu") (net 15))
 (segment (start 216.223953 33.43) (end 222.173953 33.43) (width 0.25) (layer "B.Cu") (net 15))
 (segment (start 215.22656 32.432607) (end 216.223953 33.43) (width 0.25) (layer "B.Cu") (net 15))
 (segment (start 222.173953 33.43) (end 222.541967 33.798014) (width 0.25) (layer "B.Cu") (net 15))
 (segment (start 215.22656 31.218304) (end 215.22656 32.432607) (width 0.25) (layer "B.Cu") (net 15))
 (segment (start 222.541967 33.798014) (end 222.541967 34.88441) (width 0.25) (layer "B.Cu") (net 15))
 (segment (start 216.22556 31.637213) (end 214.511967 33.350806) (width 0.25) (layer "F.Cu") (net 16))
 (segment (start 214.511967 35.25441) (end 213.421967 36.34441) (width 0.25) (layer "F.Cu") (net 16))
 (segment (start 216.22556 31.25) (end 216.22556 31.637213) (width 0.25) (layer "F.Cu") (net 16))
 (segment (start 214.511967 33.350806) (end 214.511967 35.25441) (width 0.25) (layer "F.Cu") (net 16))
 (via (at 216.22556 31.25) (size 0.8) (drill 0.4) (layers "F.Cu" "B.Cu") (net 16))
 (segment (start 216.666967 30.45941) (end 219.839759 30.45941) (width 0.25) (layer "B.Cu") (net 16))
 (segment (start 223.041967 33.661618) (end 223.041967 34.88441) (width 0.25) (layer "B.Cu") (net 16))
 (segment (start 216.22556 30.900817) (end 216.666967 30.45941) (width 0.25) (layer "B.Cu") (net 16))
 (segment (start 219.839759 30.45941) (end 223.041967 33.661618) (width 0.25) (layer "B.Cu") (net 16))
 (segment (start 216.22556 31.25) (end 216.22556 30.900817) (width 0.25) (layer "B.Cu") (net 16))
 (segment (start 212.786967 44.59941) (end 213.421967 43.96441) (width 0.4) (layer "F.Cu") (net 5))
 (segment (start 223.943967 39.261882) (end 223.943967 37.53241) (width 0.4) (layer "F.Cu") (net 5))
 (segment (start 214.706377 42.68) (end 220.525849 42.68) (width 0.4) (layer "F.Cu") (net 5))
 (segment (start 223.943967 37.53241) (end 224.813967 36.66241) (width 0.4) (layer "F.Cu") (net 5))
 (segment (start 220.525849 42.68) (end 223.943967 39.261882) (width 0.4) (layer "F.Cu") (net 5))
 (segment (start 213.421967 43.96441) (end 214.706377 42.68) (width 0.4) (layer "F.Cu") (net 5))
 (segment (start 224.813967 36.66241) (end 225.486967 36.66241) (width 0.4) (layer "F.Cu") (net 5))
 (segment (start 225.486967 36.66241) (end 224.978967 36.66241) (width 0.25) (layer "F.Cu") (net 5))
 (segment (start 200.943439 46.28441) (end 202.628439 44.59941) (width 0.4) (layer "F.Cu") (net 5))
 (segment (start 202.628439 44.59941) (end 212.786967 44.59941) (width 0.4) (layer "F.Cu") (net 5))
 (segment (start 199.791967 46.28441) (end 200.943439 46.28441) (width 0.4) (layer "F.Cu") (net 5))
 (segment (start 219.771967 44.91741) (end 219.771967 46.43441) (width 0.25) (layer "B.Cu") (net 5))
 (segment (start 219.771967 46.43441) (end 219.241967 46.96441) (width 0.25) (layer "B.Cu") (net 5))
 (segment (start 219.771967 44.91741) (end 214.374967 44.91741) (width 0.25) (layer "B.Cu") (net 5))
 (segment (start 219.241967 46.96441) (end 222.841967 46.96441) (width 0.25) (layer "B.Cu") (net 5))
 (segment (start 214.374967 44.91741) (end 213.421967 43.96441) (width 0.25) (layer "B.Cu") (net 5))
 (segment (start 218.452557 47.79941) (end 220.96 45.291967) (width 0.4) (layer "F.Cu") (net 4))
 (segment (start 209.11941 47.79941) (end 218.452557 47.79941) (width 0.4) (layer "F.Cu") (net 4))
 (segment (start 220.96 45.291967) (end 220.96 43.094377) (width 0.4) (layer "F.Cu") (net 4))
 (segment (start 208.541967 47.221967) (end 209.11941 47.79941) (width 0.4) (layer "F.Cu") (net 4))
 (segment (start 220.96 43.094377) (end 225.486967 38.56741) (width 0.4) (layer "F.Cu") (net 4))
 (segment (start 208.541967 46.34941) (end 208.541967 47.221967) (width 0.4) (layer "F.Cu") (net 4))
 (segment (start 223.866967 46.11441) (end 222.669967 44.91741) (width 0.25) (layer "B.Cu") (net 6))
 (segment (start 219.241967 48.40441) (end 222.841967 48.40441) (width 0.25) (layer "B.Cu") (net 6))
 (segment (start 222.841967 48.40441) (end 223.791967 48.40441) (width 0.25) (layer "B.Cu") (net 6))
 (segment (start 223.866967 48.32941) (end 223.866967 46.11441) (width 0.25) (layer "B.Cu") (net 6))
 (segment (start 222.669967 44.91741) (end 222.311967 44.91741) (width 0.25) (layer "B.Cu") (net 6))
 (segment (start 223.791967 48.40441) (end 223.866967 48.32941) (width 0.25) (layer "B.Cu") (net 6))
 (segment (start 205.891967 45.19941) (end 207.041967 46.34941) (width 0.4) (layer "F.Cu") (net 3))
 (segment (start 202.876967 45.19941) (end 205.891967 45.19941) (width 0.4) (layer "F.Cu") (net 3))
 (segment (start 199.791967 48.28441) (end 202.876967 45.19941) (width 0.4) (layer "F.Cu") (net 3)))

